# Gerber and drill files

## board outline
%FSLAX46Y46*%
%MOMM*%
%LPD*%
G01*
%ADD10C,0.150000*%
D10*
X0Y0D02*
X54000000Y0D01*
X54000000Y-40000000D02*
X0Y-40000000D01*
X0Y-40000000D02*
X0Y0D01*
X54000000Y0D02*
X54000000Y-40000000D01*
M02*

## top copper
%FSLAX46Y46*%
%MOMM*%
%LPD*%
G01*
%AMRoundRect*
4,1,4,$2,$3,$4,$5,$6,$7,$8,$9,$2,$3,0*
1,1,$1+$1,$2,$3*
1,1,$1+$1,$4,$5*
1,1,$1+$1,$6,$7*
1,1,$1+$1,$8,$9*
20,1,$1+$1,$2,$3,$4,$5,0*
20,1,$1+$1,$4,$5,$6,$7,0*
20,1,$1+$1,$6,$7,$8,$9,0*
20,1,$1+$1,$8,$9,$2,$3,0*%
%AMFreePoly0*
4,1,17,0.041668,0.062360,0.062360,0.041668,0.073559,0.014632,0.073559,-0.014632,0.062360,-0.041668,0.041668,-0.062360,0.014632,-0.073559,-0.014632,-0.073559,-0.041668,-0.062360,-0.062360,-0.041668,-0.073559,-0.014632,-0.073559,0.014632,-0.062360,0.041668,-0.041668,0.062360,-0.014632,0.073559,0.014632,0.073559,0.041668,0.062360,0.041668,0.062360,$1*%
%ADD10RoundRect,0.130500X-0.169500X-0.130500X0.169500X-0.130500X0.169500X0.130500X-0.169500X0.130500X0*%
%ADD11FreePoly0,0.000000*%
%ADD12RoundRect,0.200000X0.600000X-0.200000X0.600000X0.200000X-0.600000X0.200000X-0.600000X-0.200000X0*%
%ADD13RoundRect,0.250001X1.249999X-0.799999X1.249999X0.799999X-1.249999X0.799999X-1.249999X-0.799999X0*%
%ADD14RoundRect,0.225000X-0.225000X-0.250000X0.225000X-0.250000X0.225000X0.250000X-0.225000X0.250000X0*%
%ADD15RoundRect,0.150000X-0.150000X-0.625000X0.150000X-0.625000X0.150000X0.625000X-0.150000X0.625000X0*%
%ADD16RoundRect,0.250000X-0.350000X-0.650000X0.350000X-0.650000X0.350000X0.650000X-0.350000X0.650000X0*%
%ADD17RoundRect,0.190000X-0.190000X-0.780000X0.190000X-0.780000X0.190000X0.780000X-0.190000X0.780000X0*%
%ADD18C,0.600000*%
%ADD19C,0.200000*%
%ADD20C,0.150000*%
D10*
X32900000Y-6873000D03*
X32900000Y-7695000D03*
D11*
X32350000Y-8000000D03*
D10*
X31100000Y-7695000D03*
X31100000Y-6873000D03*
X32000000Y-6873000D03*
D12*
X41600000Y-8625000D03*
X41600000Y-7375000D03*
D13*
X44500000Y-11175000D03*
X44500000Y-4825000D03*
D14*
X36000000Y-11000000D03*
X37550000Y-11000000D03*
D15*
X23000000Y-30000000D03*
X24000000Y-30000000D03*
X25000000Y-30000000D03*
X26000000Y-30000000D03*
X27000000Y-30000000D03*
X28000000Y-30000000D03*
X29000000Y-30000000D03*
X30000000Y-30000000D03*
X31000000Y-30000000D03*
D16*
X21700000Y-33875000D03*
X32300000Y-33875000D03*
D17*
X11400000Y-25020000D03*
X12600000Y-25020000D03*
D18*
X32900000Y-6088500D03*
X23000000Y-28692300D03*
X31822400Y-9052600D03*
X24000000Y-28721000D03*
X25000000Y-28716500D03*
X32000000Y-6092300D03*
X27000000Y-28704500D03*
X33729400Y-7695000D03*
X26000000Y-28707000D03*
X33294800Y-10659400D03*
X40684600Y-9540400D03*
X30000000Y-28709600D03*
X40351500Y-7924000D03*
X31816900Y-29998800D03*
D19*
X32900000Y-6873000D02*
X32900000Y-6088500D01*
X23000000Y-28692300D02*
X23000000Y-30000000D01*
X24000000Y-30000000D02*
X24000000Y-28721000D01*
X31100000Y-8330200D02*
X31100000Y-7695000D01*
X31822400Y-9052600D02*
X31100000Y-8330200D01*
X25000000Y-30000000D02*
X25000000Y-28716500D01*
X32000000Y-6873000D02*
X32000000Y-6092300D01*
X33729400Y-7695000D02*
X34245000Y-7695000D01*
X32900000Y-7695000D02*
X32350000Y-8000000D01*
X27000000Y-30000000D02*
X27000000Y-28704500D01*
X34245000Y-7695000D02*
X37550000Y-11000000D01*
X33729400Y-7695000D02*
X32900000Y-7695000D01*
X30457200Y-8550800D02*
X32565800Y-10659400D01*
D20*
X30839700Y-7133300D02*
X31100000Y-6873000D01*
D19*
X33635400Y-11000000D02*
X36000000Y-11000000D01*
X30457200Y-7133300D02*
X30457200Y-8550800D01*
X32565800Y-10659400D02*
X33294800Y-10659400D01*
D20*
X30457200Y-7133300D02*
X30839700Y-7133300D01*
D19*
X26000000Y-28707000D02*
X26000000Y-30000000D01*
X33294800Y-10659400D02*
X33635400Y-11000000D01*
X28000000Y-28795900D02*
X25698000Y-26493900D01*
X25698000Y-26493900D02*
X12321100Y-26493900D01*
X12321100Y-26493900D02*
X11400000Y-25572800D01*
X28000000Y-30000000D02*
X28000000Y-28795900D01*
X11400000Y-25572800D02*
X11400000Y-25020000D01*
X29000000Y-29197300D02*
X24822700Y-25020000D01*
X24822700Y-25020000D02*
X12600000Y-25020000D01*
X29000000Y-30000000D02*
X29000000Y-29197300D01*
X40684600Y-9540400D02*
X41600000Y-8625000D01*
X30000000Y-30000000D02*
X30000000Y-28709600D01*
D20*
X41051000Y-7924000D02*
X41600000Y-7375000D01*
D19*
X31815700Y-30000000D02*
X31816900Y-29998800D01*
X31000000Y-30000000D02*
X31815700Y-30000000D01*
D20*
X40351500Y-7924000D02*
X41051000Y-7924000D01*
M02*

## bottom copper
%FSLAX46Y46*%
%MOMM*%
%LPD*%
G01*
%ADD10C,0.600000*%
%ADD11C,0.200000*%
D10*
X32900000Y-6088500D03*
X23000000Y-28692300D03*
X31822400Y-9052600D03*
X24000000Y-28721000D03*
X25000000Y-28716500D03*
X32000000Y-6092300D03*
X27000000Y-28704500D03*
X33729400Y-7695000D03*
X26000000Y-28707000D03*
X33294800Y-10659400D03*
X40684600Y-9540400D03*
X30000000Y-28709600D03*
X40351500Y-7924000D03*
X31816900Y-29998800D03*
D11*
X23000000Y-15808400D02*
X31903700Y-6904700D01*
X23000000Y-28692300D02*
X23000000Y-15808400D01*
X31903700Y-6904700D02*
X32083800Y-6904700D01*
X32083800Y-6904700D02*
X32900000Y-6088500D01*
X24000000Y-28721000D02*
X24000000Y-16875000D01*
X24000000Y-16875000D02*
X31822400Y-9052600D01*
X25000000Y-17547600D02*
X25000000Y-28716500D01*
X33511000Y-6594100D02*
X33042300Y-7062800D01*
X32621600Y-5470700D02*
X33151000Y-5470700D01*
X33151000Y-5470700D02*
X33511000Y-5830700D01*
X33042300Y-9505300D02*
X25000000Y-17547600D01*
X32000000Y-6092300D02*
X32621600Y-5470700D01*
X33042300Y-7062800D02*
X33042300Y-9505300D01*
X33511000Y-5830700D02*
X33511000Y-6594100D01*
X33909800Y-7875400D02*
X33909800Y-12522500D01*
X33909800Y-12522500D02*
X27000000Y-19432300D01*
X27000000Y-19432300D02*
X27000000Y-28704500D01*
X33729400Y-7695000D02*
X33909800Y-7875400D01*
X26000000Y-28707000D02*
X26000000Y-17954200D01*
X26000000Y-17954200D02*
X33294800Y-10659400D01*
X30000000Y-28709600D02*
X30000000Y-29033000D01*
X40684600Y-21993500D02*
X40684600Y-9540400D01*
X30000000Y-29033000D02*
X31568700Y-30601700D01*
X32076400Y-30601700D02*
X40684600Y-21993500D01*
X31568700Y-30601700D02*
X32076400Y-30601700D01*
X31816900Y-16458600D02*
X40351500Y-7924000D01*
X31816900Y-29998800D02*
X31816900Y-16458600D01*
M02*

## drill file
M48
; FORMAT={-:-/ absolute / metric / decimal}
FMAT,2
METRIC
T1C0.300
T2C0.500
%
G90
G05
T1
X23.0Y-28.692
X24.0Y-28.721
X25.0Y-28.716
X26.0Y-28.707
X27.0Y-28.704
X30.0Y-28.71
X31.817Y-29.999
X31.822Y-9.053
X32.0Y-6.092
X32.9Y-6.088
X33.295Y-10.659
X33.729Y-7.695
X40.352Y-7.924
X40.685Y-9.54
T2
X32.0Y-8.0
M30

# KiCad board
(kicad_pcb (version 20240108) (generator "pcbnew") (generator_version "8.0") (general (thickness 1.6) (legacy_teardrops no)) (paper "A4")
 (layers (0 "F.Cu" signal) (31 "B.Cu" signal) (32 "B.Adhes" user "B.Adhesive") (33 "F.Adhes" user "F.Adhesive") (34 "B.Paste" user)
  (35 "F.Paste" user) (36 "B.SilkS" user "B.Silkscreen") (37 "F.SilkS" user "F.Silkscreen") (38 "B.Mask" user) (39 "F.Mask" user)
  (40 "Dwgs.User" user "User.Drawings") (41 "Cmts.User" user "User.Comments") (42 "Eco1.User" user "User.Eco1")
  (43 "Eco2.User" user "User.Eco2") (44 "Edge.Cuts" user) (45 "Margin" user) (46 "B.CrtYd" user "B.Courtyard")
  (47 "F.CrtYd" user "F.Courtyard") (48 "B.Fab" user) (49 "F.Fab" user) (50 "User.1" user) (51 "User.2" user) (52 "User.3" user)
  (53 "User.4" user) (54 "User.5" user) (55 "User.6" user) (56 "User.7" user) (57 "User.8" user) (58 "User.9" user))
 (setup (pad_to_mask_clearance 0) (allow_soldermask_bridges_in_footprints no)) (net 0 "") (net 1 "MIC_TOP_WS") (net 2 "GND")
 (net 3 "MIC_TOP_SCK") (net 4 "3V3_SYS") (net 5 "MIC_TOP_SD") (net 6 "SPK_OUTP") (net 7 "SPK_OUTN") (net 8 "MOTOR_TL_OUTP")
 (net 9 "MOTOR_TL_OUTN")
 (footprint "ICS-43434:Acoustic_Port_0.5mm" (layer "F.Cu") (at 32 8)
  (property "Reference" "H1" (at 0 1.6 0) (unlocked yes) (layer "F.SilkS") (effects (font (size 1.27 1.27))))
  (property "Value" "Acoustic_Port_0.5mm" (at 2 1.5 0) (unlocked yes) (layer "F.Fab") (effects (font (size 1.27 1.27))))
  (pad "" np_thru_hole circle (at 0 0) (size 0.5 0.5) (drill 0.5) (layers "*.Cu" "*.Mask")))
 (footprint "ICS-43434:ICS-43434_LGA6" (layer "F.Cu") (at 32 8)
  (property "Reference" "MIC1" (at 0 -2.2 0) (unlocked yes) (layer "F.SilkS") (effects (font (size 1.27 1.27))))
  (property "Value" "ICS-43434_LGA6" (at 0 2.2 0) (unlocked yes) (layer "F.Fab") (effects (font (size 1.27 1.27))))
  (pad "1" smd roundrect (at 0.9 -1.127) (size 0.6 0.522) (layers "F.Cu" "F.Paste" "F.Mask") (roundrect_rratio 0.25) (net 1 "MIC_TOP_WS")
   (thermal_bridge_angle 45))
  (pad "2" smd roundrect (at 0.9 -0.305) (size 0.6 0.522) (layers "F.Cu" "F.Paste" "F.Mask") (roundrect_rratio 0.25) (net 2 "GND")
   (thermal_bridge_angle 45))
  (pad "3" smd custom (at 0.35 0) (size 0.15 0.15) (layers "F.Cu" "F.Mask") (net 2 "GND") (options (clearance outline) (anchor circle))
   (primitives))
  (pad "4" smd roundrect (at -0.9 -0.305) (size 0.6 0.522) (layers "F.Cu" "F.Paste" "F.Mask") (roundrect_rratio 0.25) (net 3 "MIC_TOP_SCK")
   (thermal_bridge_angle 45))
  (pad "5" smd roundrect (at -0.9 -1.127) (size 0.6 0.522) (layers "F.Cu" "F.Paste" "F.Mask") (roundrect_rratio 0.25) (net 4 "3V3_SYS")
   (thermal_bridge_angle 45))
  (pad "6" smd roundrect (at 0 -1.127) (size 0.6 0.522) (layers "F.Cu" "F.Paste" "F.Mask") (roundrect_rratio 0.25) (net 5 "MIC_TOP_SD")
   (thermal_bridge_angle 45)))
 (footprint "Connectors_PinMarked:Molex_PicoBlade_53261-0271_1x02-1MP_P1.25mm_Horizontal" (layer "F.Cu") (at 44 8 90)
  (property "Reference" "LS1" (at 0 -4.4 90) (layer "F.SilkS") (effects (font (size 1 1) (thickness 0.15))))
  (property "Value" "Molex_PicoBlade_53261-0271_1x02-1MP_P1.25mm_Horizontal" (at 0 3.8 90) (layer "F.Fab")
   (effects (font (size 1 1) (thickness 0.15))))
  (pad "1" smd roundrect (at -0.625 -2.4 90) (size 0.8 1.6) (layers "F.Cu" "F.Paste" "F.Mask") (roundrect_rratio 0.25) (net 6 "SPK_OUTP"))
  (pad "2" smd roundrect (at 0.625 -2.4 90) (size 0.8 1.6) (layers "F.Cu" "F.Paste" "F.Mask") (roundrect_rratio 0.25) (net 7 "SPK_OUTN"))
  (pad "MP" smd roundrect (at -3.175 0.5 90) (size 2.1 3) (layers "F.Cu" "F.Paste" "F.Mask") (roundrect_rratio 0.119048))
  (pad "MP" smd roundrect (at 3.175 0.5 90) (size 2.1 3) (layers "F.Cu" "F.Paste" "F.Mask") (roundrect_rratio 0.119048)))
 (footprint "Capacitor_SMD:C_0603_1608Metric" (layer "F.Cu") (at 36.775 11)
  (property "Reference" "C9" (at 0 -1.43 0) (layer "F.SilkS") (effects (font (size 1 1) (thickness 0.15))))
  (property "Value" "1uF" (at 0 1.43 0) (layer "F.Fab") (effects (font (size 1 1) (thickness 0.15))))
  (pad "1" smd roundrect (at -0.775 0) (size 0.9 0.95) (layers "F.Cu" "F.Paste" "F.Mask") (roundrect_rratio 0.25) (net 4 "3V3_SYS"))
  (pad "2" smd roundrect (at 0.775 0) (size 0.9 0.95) (layers "F.Cu" "F.Paste" "F.Mask") (roundrect_rratio 0.25) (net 2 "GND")))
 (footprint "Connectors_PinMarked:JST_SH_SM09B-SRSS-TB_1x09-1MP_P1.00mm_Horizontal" (layer "F.Cu") (at 27 32)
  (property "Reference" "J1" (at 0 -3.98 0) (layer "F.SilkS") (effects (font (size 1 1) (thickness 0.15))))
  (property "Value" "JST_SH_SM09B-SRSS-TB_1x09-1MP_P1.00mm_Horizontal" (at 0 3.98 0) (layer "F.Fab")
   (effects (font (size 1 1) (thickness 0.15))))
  (pad "1" smd roundrect (at -4 -2) (size 0.6 1.55) (layers "F.Cu" "F.Paste" "F.Mask") (roundrect_rratio 0.25) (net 1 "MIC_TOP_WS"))
  (pad "2" smd roundrect (at -3 -2) (size 0.6 1.55) (layers "F.Cu" "F.Paste" "F.Mask") (roundrect_rratio 0.25) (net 3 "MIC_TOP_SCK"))
  (pad "3" smd roundrect (at -2 -2) (size 0.6 1.55) (layers "F.Cu" "F.Paste" "F.Mask") (roundrect_rratio 0.25) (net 5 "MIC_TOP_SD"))
  (pad "4" smd roundrect (at -1 -2) (size 0.6 1.55) (layers "F.Cu" "F.Paste" "F.Mask") (roundrect_rratio 0.25) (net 4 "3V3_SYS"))
  (pad "5" smd roundrect (at 0 -2) (size 0.6 1.55) (layers "F.Cu" "F.Paste" "F.Mask") (roundrect_rratio 0.25) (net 2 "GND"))
  (pad "6" smd roundrect (at 1 -2) (size 0.6 1.55) (layers "F.Cu" "F.Paste" "F.Mask") (roundrect_rratio 0.25) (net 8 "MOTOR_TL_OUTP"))
  (pad "7" smd roundrect (at 2 -2) (size 0.6 1.55) (layers "F.Cu" "F.Paste" "F.Mask") (roundrect_rratio 0.25) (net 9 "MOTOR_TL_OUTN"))
  (pad "8" smd roundrect (at 3 -2) (size 0.6 1.55) (layers "F.Cu" "F.Paste" "F.Mask") (roundrect_rratio 0.25) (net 6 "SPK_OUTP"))
  (pad "9" smd roundrect (at 4 -2) (size 0.6 1.55) (layers "F.Cu" "F.Paste" "F.Mask") (roundrect_rratio 0.25) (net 7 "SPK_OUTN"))
  (pad "MP" smd roundrect (at -5.3 1.875) (size 1.2 1.8) (layers "F.Cu" "F.Paste" "F.Mask") (roundrect_rratio 0.208333))
  (pad "MP" smd roundrect (at 5.3 1.875) (size 1.2 1.8) (layers "F.Cu" "F.Paste" "F.Mask") (roundrect_rratio 0.208333)))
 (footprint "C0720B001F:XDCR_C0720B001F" (layer "F.Cu") (at 12 20)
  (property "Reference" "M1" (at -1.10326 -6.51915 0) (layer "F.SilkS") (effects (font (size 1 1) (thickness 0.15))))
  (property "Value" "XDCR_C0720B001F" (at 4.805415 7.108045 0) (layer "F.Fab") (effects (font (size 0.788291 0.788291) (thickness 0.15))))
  (pad "1" smd roundrect (at -0.6 5.02) (size 0.76 1.94) (layers "F.Cu" "F.Paste" "F.Mask") (roundrect_rratio 0.25) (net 8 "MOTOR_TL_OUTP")
   (solder_mask_margin 0.102))
  (pad "2" smd roundrect (at 0.6 5.02) (size 0.76 1.94) (layers "F.Cu" "F.Paste" "F.Mask") (roundrect_rratio 0.25) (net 9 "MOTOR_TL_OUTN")
   (solder_mask_margin 0.102)))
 (gr_line (start 0 0) (end 54 0) (stroke (width 0.15) (type default)) (layer "Edge.Cuts"))
 (gr_line (start 54 40) (end 0 40) (stroke (width 0.15) (type default)) (layer "Edge.Cuts"))
 (gr_line (start 0 40) (end 0 0) (stroke (width 0.15) (type default)) (layer "Edge.Cuts"))
 (gr_line (start 54 0) (end 54 40) (stroke (width 0.15) (type default)) (layer "Edge.Cuts"))
 (segment (start 32.9 6.873) (end 32.9 6.0885) (width 0.2) (layer "F.Cu") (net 1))
 (segment (start 23 28.6923) (end 23 30) (width 0.2) (layer "F.Cu") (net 1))
 (via (at 32.9 6.0885) (size 0.6) (drill 0.3) (layers "F.Cu" "B.Cu") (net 1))
 (via (at 23 28.6923) (size 0.6) (drill 0.3) (layers "F.Cu" "B.Cu") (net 1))
 (segment (start 23 15.8084) (end 31.9037 6.9047) (width 0.2) (layer "B.Cu") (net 1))
 (segment (start 23 28.6923) (end 23 15.8084) (width 0.2) (layer "B.Cu") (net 1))
 (segment (start 31.9037 6.9047) (end 32.0838 6.9047) (width 0.2) (layer "B.Cu") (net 1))
 (segment (start 32.0838 6.9047) (end 32.9 6.0885) (width 0.2) (layer "B.Cu") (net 1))
 (segment (start 24 30) (end 24 28.721) (width 0.2) (layer "F.Cu") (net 3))
 (segment (start 31.1 8.3302) (end 31.1 7.695) (width 0.2) (layer "F.Cu") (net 3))
 (segment (start 31.8224 9.0526) (end 31.1 8.3302) (width 0.2) (layer "F.Cu") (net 3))
 (via (at 31.8224 9.0526) (size 0.6) (drill 0.3) (layers "F.Cu" "B.Cu") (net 3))
 (via (at 24 28.721) (size 0.6) (drill 0.3) (layers "F.Cu" "B.Cu") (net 3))
 (segment (start 24 28.721) (end 24 16.875) (width 0.2) (layer "B.Cu") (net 3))
 (segment (start 24 16.875) (end 31.8224 9.0526) (width 0.2) (layer "B.Cu") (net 3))
 (segment (start 25 30) (end 25 28.7165) (width 0.2) (layer "F.Cu") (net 5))
 (segment (start 32 6.873) (end 32 6.0923) (width 0.2) (layer "F.Cu") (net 5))
 (via (at 25 28.7165) (size 0.6) (drill 0.3) (layers "F.Cu" "B.Cu") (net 5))
 (via (at 32 6.0923) (size 0.6) (drill 0.3) (layers "F.Cu" "B.Cu") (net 5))
 (segment (start 25 17.5476) (end 25 28.7165) (width 0.2) (layer "B.Cu") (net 5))
 (segment (start 33.511 6.5941) (end 33.0423 7.0628) (width 0.2) (layer "B.Cu") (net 5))
 (segment (start 32.6216 5.4707) (end 33.151 5.4707) (width 0.2) (layer "B.Cu") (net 5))
 (segment (start 33.151 5.4707) (end 33.511 5.8307) (width 0.2) (layer "B.Cu") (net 5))
 (segment (start 33.0423 9.5053) (end 25 17.5476) (width 0.2) (layer "B.Cu") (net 5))
 (segment (start 32 6.0923) (end 32.6216 5.4707) (width 0.2) (layer "B.Cu") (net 5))
 (segment (start 33.0423 7.0628) (end 33.0423 9.5053) (width 0.2) (layer "B.Cu") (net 5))
 (segment (start 33.511 5.8307) (end 33.511 6.5941) (width 0.2) (layer "B.Cu") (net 5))
 (segment (start 33.7294 7.695) (end 34.245 7.695) (width 0.2) (layer "F.Cu") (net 2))
 (segment (start 32.9 7.695) (end 32.35 8) (width 0.2) (layer "F.Cu") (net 2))
 (segment (start 27 30) (end 27 28.7045) (width 0.2) (layer "F.Cu") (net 2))
 (segment (start 34.245 7.695) (end 37.55 11) (width 0.2) (layer "F.Cu") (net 2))
 (segment (start 33.7294 7.695) (end 32.9 7.695) (width 0.2) (layer "F.Cu") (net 2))
 (via (at 27 28.7045) (size 0.6) (drill 0.3) (layers "F.Cu" "B.Cu") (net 2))
 (via (at 33.7294 7.695) (size 0.6) (drill 0.3) (layers "F.Cu" "B.Cu") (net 2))
 (segment (start 33.9098 7.8754) (end 33.9098 12.5225) (width 0.2) (layer "B.Cu") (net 2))
 (segment (start 33.9098 12.5225) (end 27 19.4323) (width 0.2) (layer "B.Cu") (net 2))
 (segment (start 27 19.4323) (end 27 28.7045) (width 0.2) (layer "B.Cu") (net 2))
 (segment (start 33.7294 7.695) (end 33.9098 7.8754) (width 0.2) (layer "B.Cu") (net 2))
 (segment (start 30.4572 8.5508) (end 32.5658 10.6594) (width 0.2) (layer "F.Cu") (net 4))
 (segment (start 30.8397 7.1333) (end 31.1 6.873) (width 0.15) (layer "F.Cu") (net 4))
 (segment (start 33.6354 11) (end 36 11) (width 0.2) (layer "F.Cu") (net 4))
 (segment (start 30.4572 7.1333) (end 30.4572 8.5508) (width 0.2) (layer "F.Cu") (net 4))
 (segment (start 32.5658 10.6594) (end 33.2948 10.6594) (width 0.2) (layer "F.Cu") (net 4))
 (segment (start 30.4572 7.1333) (end 30.8397 7.1333) (width 0.15) (layer "F.Cu") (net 4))
 (segment (start 26 28.707) (end 26 30) (width 0.2) (layer "F.Cu") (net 4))
 (segment (start 33.2948 10.6594) (end 33.6354 11) (width 0.2) (layer "F.Cu") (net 4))
 (via (at 26 28.707) (size 0.6) (drill 0.3) (layers "F.Cu" "B.Cu") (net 4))
 (via (at 33.2948 10.6594) (size 0.6) (drill 0.3) (layers "F.Cu" "B.Cu") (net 4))
 (segment (start 26 28.707) (end 26 17.9542) (width 0.2) (layer "B.Cu") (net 4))
 (segment (start 26 17.9542) (end 33.2948 10.6594) (width 0.2) (layer "B.Cu") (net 4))
 (segment (start 28 28.7959) (end 25.698 26.4939) (width 0.2) (layer "F.Cu") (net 8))
 (segment (start 25.698 26.4939) (end 12.3211 26.4939) (width 0.2) (layer "F.Cu") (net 8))
 (segment (start 12.3211 26.4939) (end 11.4 25.5728) (width 0.2) (layer "F.Cu") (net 8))
 (segment (start 28 30) (end 28 28.7959) (width 0.2) (layer "F.Cu") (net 8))
 (segment (start 11.4 25.5728) (end 11.4 25.02) (width 0.2) (layer "F.Cu") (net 8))
 (segment (start 29 29.1973) (end 24.8227 25.02) (width 0.2) (layer "F.Cu") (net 9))
 (segment (start 24.8227 25.02) (end 12.6 25.02) (width 0.2) (layer "F.Cu") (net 9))
 (segment (start 29 30) (end 29 29.1973) (width 0.2) (layer "F.Cu") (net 9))
 (segment (start 40.6846 9.5404) (end 41.6 8.625) (width 0.2) (layer "F.Cu") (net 6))
 (segment (start 30 30) (end 30 28.7096) (width 0.2) (layer "F.Cu") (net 6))
 (via (at 40.6846 9.5404) (size 0.6) (drill 0.3) (layers "F.Cu" "B.Cu") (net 6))
 (via (at 30 28.7096) (size 0.6) (drill 0.3) (layers "F.Cu" "B.Cu") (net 6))
 (segment (start 30 28.7096) (end 30 29.033) (width 0.2) (layer "B.Cu") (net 6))
 (segment (start 40.6846 21.9935) (end 40.6846 9.5404) (width 0.2) (layer "B.Cu") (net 6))
 (segment (start 30 29.033) (end 31.5687 30.6017) (width 0.2) (layer "B.Cu") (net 6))
 (segment (start 32.0764 30.6017) (end 40.6846 21.9935) (width 0.2) (layer "B.Cu") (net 6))
 (segment (start 31.5687 30.6017) (end 32.0764 30.6017) (width 0.2) (layer "B.Cu") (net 6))
 (segment (start 41.051 7.924) (end 41.6 7.375) (width 0.15) (layer "F.Cu") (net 7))
 (segment (start 31.8157 30) (end 31.8169 29.9988) (width 0.2) (layer "F.Cu") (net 7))
 (segment (start 31 30) (end 31.8157 30) (width 0.2) (layer "F.Cu") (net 7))
 (segment (start 40.3515 7.924) (end 41.051 7.924) (width 0.15) (layer "F.Cu") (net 7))
 (via (at 40.3515 7.924) (size 0.6) (drill 0.3) (layers "F.Cu" "B.Cu") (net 7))
 (via (at 31.8169 29.9988) (size 0.6) (drill 0.3) (layers "F.Cu" "B.Cu") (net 7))
 (segment (start 31.8169 16.4586) (end 40.3515 7.924) (width 0.2) (layer "B.Cu") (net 7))
 (segment (start 31.8169 29.9988) (end 31.8169 16.4586) (width 0.2) (layer "B.Cu") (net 7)))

